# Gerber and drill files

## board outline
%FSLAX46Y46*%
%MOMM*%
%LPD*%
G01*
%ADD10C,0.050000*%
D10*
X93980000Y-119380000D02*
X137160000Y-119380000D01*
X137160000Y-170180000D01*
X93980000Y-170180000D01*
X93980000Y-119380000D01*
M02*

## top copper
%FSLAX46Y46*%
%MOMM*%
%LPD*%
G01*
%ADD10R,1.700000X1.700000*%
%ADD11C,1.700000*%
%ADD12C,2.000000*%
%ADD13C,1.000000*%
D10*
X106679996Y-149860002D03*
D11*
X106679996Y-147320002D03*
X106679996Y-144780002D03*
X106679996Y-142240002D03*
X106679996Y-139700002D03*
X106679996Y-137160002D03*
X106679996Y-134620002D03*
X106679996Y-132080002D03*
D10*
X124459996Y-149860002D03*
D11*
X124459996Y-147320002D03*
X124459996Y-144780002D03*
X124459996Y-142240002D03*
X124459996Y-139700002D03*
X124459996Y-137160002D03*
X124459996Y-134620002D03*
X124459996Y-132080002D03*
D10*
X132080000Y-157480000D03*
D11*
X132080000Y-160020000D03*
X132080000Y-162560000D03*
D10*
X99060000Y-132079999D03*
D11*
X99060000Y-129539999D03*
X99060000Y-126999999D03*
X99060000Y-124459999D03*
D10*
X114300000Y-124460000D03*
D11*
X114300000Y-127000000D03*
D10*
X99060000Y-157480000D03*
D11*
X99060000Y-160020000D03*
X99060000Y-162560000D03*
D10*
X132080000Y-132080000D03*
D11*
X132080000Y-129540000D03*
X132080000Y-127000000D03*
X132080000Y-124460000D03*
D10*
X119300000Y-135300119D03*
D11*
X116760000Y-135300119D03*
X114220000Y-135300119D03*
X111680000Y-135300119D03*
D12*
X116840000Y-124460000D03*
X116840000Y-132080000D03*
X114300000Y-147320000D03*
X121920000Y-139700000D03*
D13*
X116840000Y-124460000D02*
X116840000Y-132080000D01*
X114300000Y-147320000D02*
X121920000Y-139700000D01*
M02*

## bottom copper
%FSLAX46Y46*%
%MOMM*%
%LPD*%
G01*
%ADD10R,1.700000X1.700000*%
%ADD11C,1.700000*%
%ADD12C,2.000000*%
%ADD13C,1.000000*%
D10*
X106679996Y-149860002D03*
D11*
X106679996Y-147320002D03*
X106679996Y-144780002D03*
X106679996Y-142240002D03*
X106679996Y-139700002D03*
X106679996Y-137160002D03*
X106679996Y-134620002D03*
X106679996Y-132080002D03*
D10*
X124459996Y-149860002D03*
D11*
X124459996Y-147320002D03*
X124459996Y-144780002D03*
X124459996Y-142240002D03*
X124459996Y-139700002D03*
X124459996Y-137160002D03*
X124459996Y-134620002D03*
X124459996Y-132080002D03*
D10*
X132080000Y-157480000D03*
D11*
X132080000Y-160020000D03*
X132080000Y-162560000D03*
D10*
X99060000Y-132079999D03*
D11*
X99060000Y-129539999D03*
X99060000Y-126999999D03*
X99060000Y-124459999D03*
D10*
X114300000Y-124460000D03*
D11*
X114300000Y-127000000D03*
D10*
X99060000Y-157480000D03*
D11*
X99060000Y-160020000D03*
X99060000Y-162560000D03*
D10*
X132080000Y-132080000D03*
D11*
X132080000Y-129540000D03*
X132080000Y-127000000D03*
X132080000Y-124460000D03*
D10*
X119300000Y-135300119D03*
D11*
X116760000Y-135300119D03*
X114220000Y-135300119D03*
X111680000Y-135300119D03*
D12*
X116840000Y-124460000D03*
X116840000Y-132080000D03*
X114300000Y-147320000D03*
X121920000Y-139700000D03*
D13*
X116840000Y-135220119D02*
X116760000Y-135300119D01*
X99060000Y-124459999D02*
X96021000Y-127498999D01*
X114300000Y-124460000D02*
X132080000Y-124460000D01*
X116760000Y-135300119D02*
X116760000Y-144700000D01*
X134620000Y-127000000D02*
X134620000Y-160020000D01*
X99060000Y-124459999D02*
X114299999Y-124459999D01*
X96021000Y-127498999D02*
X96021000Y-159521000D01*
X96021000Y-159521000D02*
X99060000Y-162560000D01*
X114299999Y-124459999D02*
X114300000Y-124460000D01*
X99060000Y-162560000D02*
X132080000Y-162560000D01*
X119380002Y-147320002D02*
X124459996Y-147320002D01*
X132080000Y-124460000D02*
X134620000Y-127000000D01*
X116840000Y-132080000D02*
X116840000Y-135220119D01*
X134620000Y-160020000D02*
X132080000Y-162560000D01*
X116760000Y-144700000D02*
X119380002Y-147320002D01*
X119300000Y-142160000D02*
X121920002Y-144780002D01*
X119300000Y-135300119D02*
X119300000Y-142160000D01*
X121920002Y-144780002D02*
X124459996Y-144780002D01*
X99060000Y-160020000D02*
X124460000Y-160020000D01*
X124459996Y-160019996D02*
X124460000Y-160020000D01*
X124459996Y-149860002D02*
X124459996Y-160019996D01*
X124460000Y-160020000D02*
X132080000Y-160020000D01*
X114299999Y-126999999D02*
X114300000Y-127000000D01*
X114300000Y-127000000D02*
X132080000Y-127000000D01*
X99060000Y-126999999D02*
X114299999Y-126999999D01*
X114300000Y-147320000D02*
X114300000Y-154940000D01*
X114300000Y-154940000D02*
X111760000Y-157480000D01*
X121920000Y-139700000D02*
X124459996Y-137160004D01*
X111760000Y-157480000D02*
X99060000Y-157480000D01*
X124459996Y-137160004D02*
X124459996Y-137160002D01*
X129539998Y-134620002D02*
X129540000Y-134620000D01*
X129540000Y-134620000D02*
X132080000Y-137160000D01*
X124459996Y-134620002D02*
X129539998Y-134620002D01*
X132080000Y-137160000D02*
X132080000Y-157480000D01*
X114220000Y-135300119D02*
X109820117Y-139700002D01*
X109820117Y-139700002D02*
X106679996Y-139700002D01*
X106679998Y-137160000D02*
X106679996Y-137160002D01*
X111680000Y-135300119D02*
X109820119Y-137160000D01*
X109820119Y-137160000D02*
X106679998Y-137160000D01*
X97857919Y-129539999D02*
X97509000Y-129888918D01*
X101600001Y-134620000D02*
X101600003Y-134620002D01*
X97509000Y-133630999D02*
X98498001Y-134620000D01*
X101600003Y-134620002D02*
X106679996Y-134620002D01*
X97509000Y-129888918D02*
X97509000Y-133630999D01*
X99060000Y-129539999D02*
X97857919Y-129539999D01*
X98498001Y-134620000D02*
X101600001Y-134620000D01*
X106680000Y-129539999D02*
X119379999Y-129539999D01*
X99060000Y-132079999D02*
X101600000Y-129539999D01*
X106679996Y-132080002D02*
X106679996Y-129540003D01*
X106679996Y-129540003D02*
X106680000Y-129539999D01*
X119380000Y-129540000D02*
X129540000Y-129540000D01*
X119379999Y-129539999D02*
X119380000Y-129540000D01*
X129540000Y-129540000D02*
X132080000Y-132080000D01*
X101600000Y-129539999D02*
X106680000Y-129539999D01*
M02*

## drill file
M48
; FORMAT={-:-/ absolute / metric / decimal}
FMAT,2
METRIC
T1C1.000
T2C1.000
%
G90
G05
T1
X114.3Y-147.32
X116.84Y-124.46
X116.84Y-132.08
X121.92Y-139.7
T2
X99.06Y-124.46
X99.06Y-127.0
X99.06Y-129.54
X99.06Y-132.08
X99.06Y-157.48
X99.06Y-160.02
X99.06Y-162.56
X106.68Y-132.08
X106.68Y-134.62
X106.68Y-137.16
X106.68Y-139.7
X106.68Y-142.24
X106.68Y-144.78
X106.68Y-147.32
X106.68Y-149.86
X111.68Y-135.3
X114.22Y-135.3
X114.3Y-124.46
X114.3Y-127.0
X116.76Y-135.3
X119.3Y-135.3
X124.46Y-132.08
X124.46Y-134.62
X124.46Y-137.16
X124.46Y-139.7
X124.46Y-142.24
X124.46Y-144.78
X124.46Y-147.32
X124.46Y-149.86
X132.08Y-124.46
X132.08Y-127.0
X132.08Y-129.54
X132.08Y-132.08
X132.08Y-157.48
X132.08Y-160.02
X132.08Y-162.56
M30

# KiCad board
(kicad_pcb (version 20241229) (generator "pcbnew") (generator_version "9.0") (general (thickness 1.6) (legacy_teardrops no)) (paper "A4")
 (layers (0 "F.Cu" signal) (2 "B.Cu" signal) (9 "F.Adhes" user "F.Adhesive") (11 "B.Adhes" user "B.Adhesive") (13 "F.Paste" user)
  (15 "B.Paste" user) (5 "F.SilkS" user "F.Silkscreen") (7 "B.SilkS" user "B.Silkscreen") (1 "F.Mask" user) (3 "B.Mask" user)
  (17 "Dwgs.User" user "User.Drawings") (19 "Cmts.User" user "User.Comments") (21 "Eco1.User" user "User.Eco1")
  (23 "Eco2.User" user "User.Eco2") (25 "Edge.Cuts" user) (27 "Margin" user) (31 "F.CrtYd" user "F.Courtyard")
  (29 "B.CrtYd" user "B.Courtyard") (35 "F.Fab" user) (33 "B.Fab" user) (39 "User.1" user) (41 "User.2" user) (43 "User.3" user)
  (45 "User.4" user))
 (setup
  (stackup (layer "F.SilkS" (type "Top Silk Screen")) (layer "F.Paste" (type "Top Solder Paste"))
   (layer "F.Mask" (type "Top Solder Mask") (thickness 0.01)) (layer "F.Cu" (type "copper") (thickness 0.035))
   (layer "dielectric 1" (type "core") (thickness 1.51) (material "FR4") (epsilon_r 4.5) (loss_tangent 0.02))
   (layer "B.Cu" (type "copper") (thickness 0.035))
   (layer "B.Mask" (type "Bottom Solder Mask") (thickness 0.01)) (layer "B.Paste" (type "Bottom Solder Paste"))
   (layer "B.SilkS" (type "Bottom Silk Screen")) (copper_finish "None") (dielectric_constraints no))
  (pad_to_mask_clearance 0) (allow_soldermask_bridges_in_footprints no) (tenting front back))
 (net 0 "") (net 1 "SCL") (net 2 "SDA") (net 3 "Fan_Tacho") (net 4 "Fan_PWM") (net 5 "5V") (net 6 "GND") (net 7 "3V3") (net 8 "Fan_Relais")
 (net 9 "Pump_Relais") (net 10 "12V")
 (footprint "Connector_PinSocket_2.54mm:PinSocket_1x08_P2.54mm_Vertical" (layer "F.Cu") (at 106.679996 149.860002 180)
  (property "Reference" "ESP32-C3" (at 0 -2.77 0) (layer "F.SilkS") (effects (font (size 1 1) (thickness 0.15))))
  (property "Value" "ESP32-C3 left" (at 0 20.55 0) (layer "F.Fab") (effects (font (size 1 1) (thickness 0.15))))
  (pad "1" thru_hole rect (at 0 0 180) (size 1.7 1.7) (drill 1) (layers "*.Cu" "*.Mask") (remove_unused_layers no))
  (pad "2" thru_hole circle (at 0 2.54 180) (size 1.7 1.7) (drill 1) (layers "*.Cu" "*.Mask") (remove_unused_layers no))
  (pad "3" thru_hole circle (at 0 5.08 180) (size 1.7 1.7) (drill 1) (layers "*.Cu" "*.Mask") (remove_unused_layers no))
  (pad "4" thru_hole circle (at 0 7.62 180) (size 1.7 1.7) (drill 1) (layers "*.Cu" "*.Mask") (remove_unused_layers no))
  (pad "5" thru_hole circle (at 0 10.16 180) (size 1.7 1.7) (drill 1) (layers "*.Cu" "*.Mask") (remove_unused_layers no) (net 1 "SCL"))
  (pad "6" thru_hole circle (at 0 12.7 180) (size 1.7 1.7) (drill 1) (layers "*.Cu" "*.Mask") (remove_unused_layers no) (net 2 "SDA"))
  (pad "7" thru_hole circle (at 0 15.24 180) (size 1.7 1.7) (drill 1) (layers "*.Cu" "*.Mask") (remove_unused_layers no) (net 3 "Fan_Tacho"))
  (pad "8" thru_hole circle (at 0 17.78 180) (size 1.7 1.7) (drill 1) (layers "*.Cu" "*.Mask") (remove_unused_layers no) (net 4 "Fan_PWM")))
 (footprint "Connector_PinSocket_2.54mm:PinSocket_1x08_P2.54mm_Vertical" (layer "F.Cu") (at 124.459996 149.860002 180)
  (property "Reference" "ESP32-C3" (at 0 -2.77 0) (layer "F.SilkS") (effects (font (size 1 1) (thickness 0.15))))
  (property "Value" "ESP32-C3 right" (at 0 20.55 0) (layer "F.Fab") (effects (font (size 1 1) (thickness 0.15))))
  (pad "1" thru_hole rect (at 0 0 180) (size 1.7 1.7) (drill 1) (layers "*.Cu" "*.Mask") (remove_unused_layers no) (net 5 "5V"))
  (pad "2" thru_hole circle (at 0 2.54 180) (size 1.7 1.7) (drill 1) (layers "*.Cu" "*.Mask") (remove_unused_layers no) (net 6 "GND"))
  (pad "3" thru_hole circle (at 0 5.08 180) (size 1.7 1.7) (drill 1) (layers "*.Cu" "*.Mask") (remove_unused_layers no) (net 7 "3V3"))
  (pad "4" thru_hole circle (at 0 7.62 180) (size 1.7 1.7) (drill 1) (layers "*.Cu" "*.Mask") (remove_unused_layers no))
  (pad "5" thru_hole circle (at 0 10.16 180) (size 1.7 1.7) (drill 1) (layers "*.Cu" "*.Mask") (remove_unused_layers no))
  (pad "6" thru_hole circle (at 0 12.7 180) (size 1.7 1.7) (drill 1) (layers "*.Cu" "*.Mask") (remove_unused_layers no) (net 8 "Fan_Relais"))
  (pad "7" thru_hole circle (at 0 15.24 180) (size 1.7 1.7) (drill 1) (layers "*.Cu" "*.Mask") (remove_unused_layers no)
   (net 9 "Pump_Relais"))
  (pad "8" thru_hole circle (at 0 17.78 180) (size 1.7 1.7) (drill 1) (layers "*.Cu" "*.Mask") (remove_unused_layers no)))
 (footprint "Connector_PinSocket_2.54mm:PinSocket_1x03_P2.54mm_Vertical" (layer "B.Cu") (at 132.08 157.48 180)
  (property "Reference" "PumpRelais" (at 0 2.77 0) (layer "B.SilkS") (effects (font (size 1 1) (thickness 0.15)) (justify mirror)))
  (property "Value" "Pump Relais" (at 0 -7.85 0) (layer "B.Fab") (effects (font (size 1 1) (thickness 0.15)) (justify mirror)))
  (pad "1" thru_hole rect (at 0 0 180) (size 1.7 1.7) (drill 1) (layers "*.Cu" "*.Mask") (remove_unused_layers no) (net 9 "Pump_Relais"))
  (pad "2" thru_hole circle (at 0 -2.54 180) (size 1.7 1.7) (drill 1) (layers "*.Cu" "*.Mask") (remove_unused_layers no) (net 5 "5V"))
  (pad "3" thru_hole circle (at 0 -5.08 180) (size 1.7 1.7) (drill 1) (layers "*.Cu" "*.Mask") (remove_unused_layers no) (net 6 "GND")))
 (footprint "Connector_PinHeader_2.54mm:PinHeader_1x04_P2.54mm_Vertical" (layer "B.Cu") (at 99.06 132.079999)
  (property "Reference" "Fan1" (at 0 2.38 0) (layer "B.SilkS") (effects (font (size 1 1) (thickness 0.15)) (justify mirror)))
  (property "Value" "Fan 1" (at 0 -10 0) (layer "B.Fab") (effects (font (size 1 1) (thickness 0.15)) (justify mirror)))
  (pad "1" thru_hole rect (at 0 0) (size 1.7 1.7) (drill 1) (layers "*.Cu" "*.Mask") (remove_unused_layers no) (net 4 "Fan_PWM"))
  (pad "2" thru_hole circle (at 0 -2.54) (size 1.7 1.7) (drill 1) (layers "*.Cu" "*.Mask") (remove_unused_layers no) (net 3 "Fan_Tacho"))
  (pad "3" thru_hole circle (at 0 -5.08) (size 1.7 1.7) (drill 1) (layers "*.Cu" "*.Mask") (remove_unused_layers no) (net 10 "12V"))
  (pad "4" thru_hole circle (at 0 -7.62) (size 1.7 1.7) (drill 1) (layers "*.Cu" "*.Mask") (remove_unused_layers no) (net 6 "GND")))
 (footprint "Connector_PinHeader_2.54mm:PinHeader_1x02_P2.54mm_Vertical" (layer "B.Cu") (at 114.3 124.46 180)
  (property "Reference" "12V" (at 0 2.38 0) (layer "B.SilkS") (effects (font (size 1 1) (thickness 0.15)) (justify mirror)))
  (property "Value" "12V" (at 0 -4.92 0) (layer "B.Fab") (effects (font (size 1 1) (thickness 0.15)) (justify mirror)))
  (pad "1" thru_hole rect (at 0 0 180) (size 1.7 1.7) (drill 1) (layers "*.Cu" "*.Mask") (remove_unused_layers no) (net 6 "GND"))
  (pad "2" thru_hole circle (at 0 -2.54 180) (size 1.7 1.7) (drill 1) (layers "*.Cu" "*.Mask") (remove_unused_layers no) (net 10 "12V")))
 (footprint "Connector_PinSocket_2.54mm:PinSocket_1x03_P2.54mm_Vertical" (layer "B.Cu") (at 99.06 157.48 180)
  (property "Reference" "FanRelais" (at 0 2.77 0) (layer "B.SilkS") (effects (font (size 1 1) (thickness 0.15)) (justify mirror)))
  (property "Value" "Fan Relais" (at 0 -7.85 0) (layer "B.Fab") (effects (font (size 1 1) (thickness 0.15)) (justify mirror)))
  (pad "1" thru_hole rect (at 0 0 180) (size 1.7 1.7) (drill 1) (layers "*.Cu" "*.Mask") (remove_unused_layers no) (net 8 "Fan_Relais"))
  (pad "2" thru_hole circle (at 0 -2.54 180) (size 1.7 1.7) (drill 1) (layers "*.Cu" "*.Mask") (remove_unused_layers no) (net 5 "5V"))
  (pad "3" thru_hole circle (at 0 -5.08 180) (size 1.7 1.7) (drill 1) (layers "*.Cu" "*.Mask") (remove_unused_layers no) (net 6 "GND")))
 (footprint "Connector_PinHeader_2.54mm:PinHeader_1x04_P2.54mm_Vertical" (layer "B.Cu") (at 132.08 132.08)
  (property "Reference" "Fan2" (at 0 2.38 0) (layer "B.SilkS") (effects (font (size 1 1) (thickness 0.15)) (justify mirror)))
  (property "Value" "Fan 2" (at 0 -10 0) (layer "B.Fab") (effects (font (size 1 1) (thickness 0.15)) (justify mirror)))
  (pad "1" thru_hole rect (at 0 0) (size 1.7 1.7) (drill 1) (layers "*.Cu" "*.Mask") (remove_unused_layers no) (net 4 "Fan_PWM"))
  (pad "2" thru_hole circle (at 0 -2.54) (size 1.7 1.7) (drill 1) (layers "*.Cu" "*.Mask") (remove_unused_layers no))
  (pad "3" thru_hole circle (at 0 -5.08) (size 1.7 1.7) (drill 1) (layers "*.Cu" "*.Mask") (remove_unused_layers no) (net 10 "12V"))
  (pad "4" thru_hole circle (at 0 -7.62) (size 1.7 1.7) (drill 1) (layers "*.Cu" "*.Mask") (remove_unused_layers no) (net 6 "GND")))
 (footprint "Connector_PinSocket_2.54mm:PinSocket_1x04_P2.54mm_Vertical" (layer "B.Cu") (at 119.3 135.300119 90)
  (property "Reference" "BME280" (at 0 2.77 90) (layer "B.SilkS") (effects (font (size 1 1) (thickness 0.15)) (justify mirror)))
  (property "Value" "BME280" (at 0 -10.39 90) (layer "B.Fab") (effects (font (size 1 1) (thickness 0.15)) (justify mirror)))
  (pad "1" thru_hole rect (at 0 0 90) (size 1.7 1.7) (drill 1) (layers "*.Cu" "*.Mask") (remove_unused_layers no) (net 7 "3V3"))
  (pad "2" thru_hole circle (at 0 -2.54 90) (size 1.7 1.7) (drill 1) (layers "*.Cu" "*.Mask") (remove_unused_layers no) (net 6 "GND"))
  (pad "3" thru_hole circle (at 0 -5.08 90) (size 1.7 1.7) (drill 1) (layers "*.Cu" "*.Mask") (remove_unused_layers no) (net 1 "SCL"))
  (pad "4" thru_hole circle (at 0 -7.62 90) (size 1.7 1.7) (drill 1) (layers "*.Cu" "*.Mask") (remove_unused_layers no) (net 2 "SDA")))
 (gr_rect (start 93.98 119.38) (end 137.16 170.18) (stroke (width 0.05) (type default)) (fill no) (layer "Edge.Cuts"))
 (segment (start 116.84 124.46) (end 116.84 132.08) (width 1) (layer "F.Cu") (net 6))
 (via (at 116.84 124.46) (size 2) (drill 1) (layers "F.Cu" "B.Cu") (free yes) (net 6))
 (via (at 116.84 132.08) (size 2) (drill 1) (layers "F.Cu" "B.Cu") (free yes) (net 6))
 (segment (start 116.84 135.220119) (end 116.76 135.300119) (width 1) (layer "B.Cu") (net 6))
 (segment (start 99.06 124.459999) (end 96.021 127.498999) (width 1) (layer "B.Cu") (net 6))
 (segment (start 114.3 124.46) (end 132.08 124.46) (width 1) (layer "B.Cu") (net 6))
 (segment (start 116.76 135.300119) (end 116.76 144.7) (width 1) (layer "B.Cu") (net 6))
 (segment (start 134.62 127) (end 134.62 160.02) (width 1) (layer "B.Cu") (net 6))
 (segment (start 99.06 124.459999) (end 114.299999 124.459999) (width 1) (layer "B.Cu") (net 6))
 (segment (start 96.021 127.498999) (end 96.021 159.521) (width 1) (layer "B.Cu") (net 6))
 (segment (start 96.021 159.521) (end 99.06 162.56) (width 1) (layer "B.Cu") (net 6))
 (segment (start 114.299999 124.459999) (end 114.3 124.46) (width 1) (layer "B.Cu") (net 6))
 (segment (start 99.06 162.56) (end 132.08 162.56) (width 1) (layer "B.Cu") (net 6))
 (segment (start 119.380002 147.320002) (end 124.459996 147.320002) (width 1) (layer "B.Cu") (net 6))
 (segment (start 132.08 124.46) (end 134.62 127) (width 1) (layer "B.Cu") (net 6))
 (segment (start 116.84 132.08) (end 116.84 135.220119) (width 1) (layer "B.Cu") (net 6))
 (segment (start 134.62 160.02) (end 132.08 162.56) (width 1) (layer "B.Cu") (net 6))
 (segment (start 116.76 144.7) (end 119.380002 147.320002) (width 1) (layer "B.Cu") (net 6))
 (segment (start 119.3 142.16) (end 121.920002 144.780002) (width 1) (layer "B.Cu") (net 7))
 (segment (start 119.3 135.300119) (end 119.3 142.16) (width 1) (layer "B.Cu") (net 7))
 (segment (start 121.920002 144.780002) (end 124.459996 144.780002) (width 1) (layer "B.Cu") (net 7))
 (segment (start 99.06 160.02) (end 124.46 160.02) (width 1) (layer "B.Cu") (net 5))
 (segment (start 124.459996 160.019996) (end 124.46 160.02) (width 1) (layer "B.Cu") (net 5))
 (segment (start 124.459996 149.860002) (end 124.459996 160.019996) (width 1) (layer "B.Cu") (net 5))
 (segment (start 124.46 160.02) (end 132.08 160.02) (width 1) (layer "B.Cu") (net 5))
 (segment (start 114.299999 126.999999) (end 114.3 127) (width 1) (layer "B.Cu") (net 10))
 (segment (start 114.3 127) (end 132.08 127) (width 1) (layer "B.Cu") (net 10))
 (segment (start 99.06 126.999999) (end 114.299999 126.999999) (width 1) (layer "B.Cu") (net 10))
 (segment (start 114.3 147.32) (end 121.92 139.7) (width 1) (layer "F.Cu") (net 8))
 (via (at 114.3 147.32) (size 2) (drill 1) (layers "F.Cu" "B.Cu") (free yes) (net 8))
 (via (at 121.92 139.7) (size 2) (drill 1) (layers "F.Cu" "B.Cu") (free yes) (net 8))
 (segment (start 114.3 147.32) (end 114.3 154.94) (width 1) (layer "B.Cu") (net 8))
 (segment (start 114.3 154.94) (end 111.76 157.48) (width 1) (layer "B.Cu") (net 8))
 (segment (start 121.92 139.7) (end 124.459996 137.160004) (width 1) (layer "B.Cu") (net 8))
 (segment (start 111.76 157.48) (end 99.06 157.48) (width 1) (layer "B.Cu") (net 8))
 (segment (start 124.459996 137.160004) (end 124.459996 137.160002) (width 1) (layer "B.Cu") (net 8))
 (segment (start 129.539998 134.620002) (end 129.54 134.62) (width 1) (layer "B.Cu") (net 9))
 (segment (start 129.54 134.62) (end 132.08 137.16) (width 1) (layer "B.Cu") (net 9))
 (segment (start 124.459996 134.620002) (end 129.539998 134.620002) (width 1) (layer "B.Cu") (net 9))
 (segment (start 132.08 137.16) (end 132.08 157.48) (width 1) (layer "B.Cu") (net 9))
 (segment (start 114.22 135.300119) (end 109.820117 139.700002) (width 1) (layer "B.Cu") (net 1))
 (segment (start 109.820117 139.700002) (end 106.679996 139.700002) (width 1) (layer "B.Cu") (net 1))
 (segment (start 106.679998 137.16) (end 106.679996 137.160002) (width 1) (layer "B.Cu") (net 2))
 (segment (start 111.68 135.300119) (end 109.820119 137.16) (width 1) (layer "B.Cu") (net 2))
 (segment (start 109.820119 137.16) (end 106.679998 137.16) (width 1) (layer "B.Cu") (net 2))
 (segment (start 97.857919 129.539999) (end 97.509 129.888918) (width 1) (layer "B.Cu") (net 3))
 (segment (start 101.600001 134.62) (end 101.600003 134.620002) (width 1) (layer "B.Cu") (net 3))
 (segment (start 97.509 133.630999) (end 98.498001 134.62) (width 1) (layer "B.Cu") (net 3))
 (segment (start 101.600003 134.620002) (end 106.679996 134.620002) (width 1) (layer "B.Cu") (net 3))
 (segment (start 97.509 129.888918) (end 97.509 133.630999) (width 1) (layer "B.Cu") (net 3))
 (segment (start 99.06 129.539999) (end 97.857919 129.539999) (width 1) (layer "B.Cu") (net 3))
 (segment (start 98.498001 134.62) (end 101.600001 134.62) (width 1) (layer "B.Cu") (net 3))
 (segment (start 106.68 129.539999) (end 119.379999 129.539999) (width 1) (layer "B.Cu") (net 4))
 (segment (start 99.06 132.079999) (end 101.6 129.539999) (width 1) (layer "B.Cu") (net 4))
 (segment (start 106.679996 132.080002) (end 106.679996 129.540003) (width 1) (layer "B.Cu") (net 4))
 (segment (start 106.679996 129.540003) (end 106.68 129.539999) (width 1) (layer "B.Cu") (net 4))
 (segment (start 119.38 129.54) (end 129.54 129.54) (width 1) (layer "B.Cu") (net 4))
 (segment (start 119.379999 129.539999) (end 119.38 129.54) (width 1) (layer "B.Cu") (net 4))
 (segment (start 129.54 129.54) (end 132.08 132.08) (width 1) (layer "B.Cu") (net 4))
 (segment (start 101.6 129.539999) (end 106.68 129.539999) (width 1) (layer "B.Cu") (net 4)))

